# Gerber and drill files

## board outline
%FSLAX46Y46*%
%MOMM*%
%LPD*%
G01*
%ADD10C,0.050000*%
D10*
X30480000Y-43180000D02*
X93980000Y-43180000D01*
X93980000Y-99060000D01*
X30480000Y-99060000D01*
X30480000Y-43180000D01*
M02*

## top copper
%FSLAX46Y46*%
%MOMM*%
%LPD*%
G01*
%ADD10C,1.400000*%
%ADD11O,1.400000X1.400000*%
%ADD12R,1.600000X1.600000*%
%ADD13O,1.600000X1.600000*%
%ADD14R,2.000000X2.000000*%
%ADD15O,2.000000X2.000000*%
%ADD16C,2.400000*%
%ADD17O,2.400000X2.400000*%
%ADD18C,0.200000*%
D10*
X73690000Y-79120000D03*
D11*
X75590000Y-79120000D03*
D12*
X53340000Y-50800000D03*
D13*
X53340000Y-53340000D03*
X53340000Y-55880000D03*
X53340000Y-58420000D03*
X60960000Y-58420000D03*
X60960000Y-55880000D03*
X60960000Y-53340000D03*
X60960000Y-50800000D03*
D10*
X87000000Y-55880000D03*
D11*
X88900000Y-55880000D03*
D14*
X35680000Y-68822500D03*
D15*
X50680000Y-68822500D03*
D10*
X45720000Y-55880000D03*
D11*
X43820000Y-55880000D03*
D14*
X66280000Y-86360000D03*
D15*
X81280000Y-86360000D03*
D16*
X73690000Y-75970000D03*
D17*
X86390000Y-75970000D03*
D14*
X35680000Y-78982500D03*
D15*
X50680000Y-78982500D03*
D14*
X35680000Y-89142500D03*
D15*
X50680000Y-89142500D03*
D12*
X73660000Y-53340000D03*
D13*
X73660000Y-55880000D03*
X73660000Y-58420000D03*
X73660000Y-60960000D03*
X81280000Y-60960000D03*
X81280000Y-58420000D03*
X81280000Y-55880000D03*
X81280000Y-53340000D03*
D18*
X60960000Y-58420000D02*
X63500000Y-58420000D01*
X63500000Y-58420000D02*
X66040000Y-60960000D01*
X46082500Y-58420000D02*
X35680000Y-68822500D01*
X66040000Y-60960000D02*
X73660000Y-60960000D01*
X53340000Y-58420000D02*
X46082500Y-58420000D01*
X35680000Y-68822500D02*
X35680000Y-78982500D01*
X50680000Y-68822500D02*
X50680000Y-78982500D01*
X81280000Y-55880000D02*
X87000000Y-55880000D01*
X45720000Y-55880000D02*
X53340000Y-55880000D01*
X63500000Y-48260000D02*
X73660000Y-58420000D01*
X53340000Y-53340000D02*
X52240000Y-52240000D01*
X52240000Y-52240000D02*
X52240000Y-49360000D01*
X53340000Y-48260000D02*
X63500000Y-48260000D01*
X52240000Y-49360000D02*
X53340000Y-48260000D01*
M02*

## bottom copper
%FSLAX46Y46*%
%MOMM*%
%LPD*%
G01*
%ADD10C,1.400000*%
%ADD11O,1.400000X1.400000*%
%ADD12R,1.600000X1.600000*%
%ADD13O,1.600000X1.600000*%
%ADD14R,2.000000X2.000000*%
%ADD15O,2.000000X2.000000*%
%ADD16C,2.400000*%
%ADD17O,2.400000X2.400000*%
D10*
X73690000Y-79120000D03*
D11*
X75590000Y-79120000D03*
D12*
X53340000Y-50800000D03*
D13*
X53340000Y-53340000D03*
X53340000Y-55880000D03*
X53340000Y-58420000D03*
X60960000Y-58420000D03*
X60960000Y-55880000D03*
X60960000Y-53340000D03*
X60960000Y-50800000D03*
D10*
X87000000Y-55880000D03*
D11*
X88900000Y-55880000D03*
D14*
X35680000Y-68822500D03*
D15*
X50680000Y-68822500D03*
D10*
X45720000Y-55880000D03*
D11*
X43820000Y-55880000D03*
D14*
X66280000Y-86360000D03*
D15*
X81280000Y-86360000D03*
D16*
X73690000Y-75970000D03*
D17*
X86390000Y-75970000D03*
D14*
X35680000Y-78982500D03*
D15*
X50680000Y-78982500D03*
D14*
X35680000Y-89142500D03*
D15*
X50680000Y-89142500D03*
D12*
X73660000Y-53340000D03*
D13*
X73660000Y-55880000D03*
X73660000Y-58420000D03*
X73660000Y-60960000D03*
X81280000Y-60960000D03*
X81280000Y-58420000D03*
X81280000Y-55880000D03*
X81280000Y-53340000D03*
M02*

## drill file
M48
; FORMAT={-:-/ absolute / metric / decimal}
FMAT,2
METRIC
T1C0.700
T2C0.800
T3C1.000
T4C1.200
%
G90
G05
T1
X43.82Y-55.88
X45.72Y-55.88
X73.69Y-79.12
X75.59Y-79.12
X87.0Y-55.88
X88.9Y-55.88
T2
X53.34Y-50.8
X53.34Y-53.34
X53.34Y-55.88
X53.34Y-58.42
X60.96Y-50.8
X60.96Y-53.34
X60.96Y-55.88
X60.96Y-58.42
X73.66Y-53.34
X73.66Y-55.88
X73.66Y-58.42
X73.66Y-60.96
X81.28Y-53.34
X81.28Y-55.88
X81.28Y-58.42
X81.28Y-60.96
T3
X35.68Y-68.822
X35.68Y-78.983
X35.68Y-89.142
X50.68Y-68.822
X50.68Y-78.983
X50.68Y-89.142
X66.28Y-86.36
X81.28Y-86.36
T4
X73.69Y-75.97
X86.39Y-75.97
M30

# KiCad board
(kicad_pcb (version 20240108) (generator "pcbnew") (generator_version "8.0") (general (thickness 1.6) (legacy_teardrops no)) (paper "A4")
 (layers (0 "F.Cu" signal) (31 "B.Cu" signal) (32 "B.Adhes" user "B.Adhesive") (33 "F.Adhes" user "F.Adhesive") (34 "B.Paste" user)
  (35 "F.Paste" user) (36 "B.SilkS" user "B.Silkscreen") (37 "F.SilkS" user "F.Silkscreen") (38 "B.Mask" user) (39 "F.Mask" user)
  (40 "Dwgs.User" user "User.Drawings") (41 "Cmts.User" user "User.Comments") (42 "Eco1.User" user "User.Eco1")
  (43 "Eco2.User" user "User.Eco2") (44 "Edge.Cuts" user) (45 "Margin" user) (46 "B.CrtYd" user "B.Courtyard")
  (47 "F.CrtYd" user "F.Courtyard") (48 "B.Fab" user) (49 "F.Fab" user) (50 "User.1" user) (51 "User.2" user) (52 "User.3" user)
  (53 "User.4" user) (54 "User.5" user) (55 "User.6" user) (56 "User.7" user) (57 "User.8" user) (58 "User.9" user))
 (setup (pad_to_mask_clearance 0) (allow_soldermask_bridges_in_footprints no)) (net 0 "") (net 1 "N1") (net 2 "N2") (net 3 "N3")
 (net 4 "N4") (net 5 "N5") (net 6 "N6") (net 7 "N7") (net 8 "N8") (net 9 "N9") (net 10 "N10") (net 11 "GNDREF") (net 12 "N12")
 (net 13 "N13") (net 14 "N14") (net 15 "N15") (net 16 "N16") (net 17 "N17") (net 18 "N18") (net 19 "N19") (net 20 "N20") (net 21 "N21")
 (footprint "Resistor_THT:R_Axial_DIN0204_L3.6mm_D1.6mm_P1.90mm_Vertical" (layer "F.Cu") (at 73.69 79.12)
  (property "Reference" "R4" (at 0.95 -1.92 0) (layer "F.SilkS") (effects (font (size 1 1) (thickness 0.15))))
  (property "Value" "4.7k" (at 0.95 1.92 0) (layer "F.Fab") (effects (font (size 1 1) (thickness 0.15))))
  (pad "1" thru_hole circle (at 0 0) (size 1.4 1.4) (drill 0.7) (layers "*.Cu" "*.Mask") (remove_unused_layers no) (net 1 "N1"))
  (pad "2" thru_hole oval (at 1.9 0) (size 1.4 1.4) (drill 0.7) (layers "*.Cu" "*.Mask") (remove_unused_layers no) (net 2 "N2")))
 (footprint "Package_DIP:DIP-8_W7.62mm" (layer "F.Cu") (at 53.34 50.8)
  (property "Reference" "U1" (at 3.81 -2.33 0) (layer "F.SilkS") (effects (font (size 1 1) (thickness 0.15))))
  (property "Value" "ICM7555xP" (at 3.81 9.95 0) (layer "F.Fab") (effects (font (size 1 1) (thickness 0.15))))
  (pad "1" thru_hole rect (at 0 0) (size 1.6 1.6) (drill 0.8) (layers "*.Cu" "*.Mask") (remove_unused_layers no) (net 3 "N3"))
  (pad "2" thru_hole oval (at 0 2.54) (size 1.6 1.6) (drill 0.8) (layers "*.Cu" "*.Mask") (remove_unused_layers no) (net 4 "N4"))
  (pad "3" thru_hole oval (at 0 5.08) (size 1.6 1.6) (drill 0.8) (layers "*.Cu" "*.Mask") (remove_unused_layers no) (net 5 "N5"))
  (pad "4" thru_hole oval (at 0 7.62) (size 1.6 1.6) (drill 0.8) (layers "*.Cu" "*.Mask") (remove_unused_layers no) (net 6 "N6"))
  (pad "5" thru_hole oval (at 7.62 7.62) (size 1.6 1.6) (drill 0.8) (layers "*.Cu" "*.Mask") (remove_unused_layers no) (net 6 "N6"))
  (pad "6" thru_hole oval (at 7.62 5.08) (size 1.6 1.6) (drill 0.8) (layers "*.Cu" "*.Mask") (remove_unused_layers no) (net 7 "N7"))
  (pad "7" thru_hole oval (at 7.62 2.54) (size 1.6 1.6) (drill 0.8) (layers "*.Cu" "*.Mask") (remove_unused_layers no) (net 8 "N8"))
  (pad "8" thru_hole oval (at 7.62 0) (size 1.6 1.6) (drill 0.8) (layers "*.Cu" "*.Mask") (remove_unused_layers no) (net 6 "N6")))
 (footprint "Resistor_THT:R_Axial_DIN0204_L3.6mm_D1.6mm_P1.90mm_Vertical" (layer "F.Cu") (at 87 55.88)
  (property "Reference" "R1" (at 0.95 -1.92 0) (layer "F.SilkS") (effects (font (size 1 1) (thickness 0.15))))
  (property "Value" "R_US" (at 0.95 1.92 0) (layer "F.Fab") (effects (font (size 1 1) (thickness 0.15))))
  (pad "1" thru_hole circle (at 0 0) (size 1.4 1.4) (drill 0.7) (layers "*.Cu" "*.Mask") (remove_unused_layers no) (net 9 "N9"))
  (pad "2" thru_hole oval (at 1.9 0) (size 1.4 1.4) (drill 0.7) (layers "*.Cu" "*.Mask") (remove_unused_layers no) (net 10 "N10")))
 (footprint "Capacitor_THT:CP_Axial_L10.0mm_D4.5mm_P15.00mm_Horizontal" (layer "F.Cu") (at 35.68 68.8225)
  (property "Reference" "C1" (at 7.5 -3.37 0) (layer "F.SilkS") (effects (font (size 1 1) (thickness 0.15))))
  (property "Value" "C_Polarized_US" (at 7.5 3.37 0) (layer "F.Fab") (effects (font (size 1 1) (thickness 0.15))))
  (pad "1" thru_hole rect (at 0 0) (size 2 2) (drill 1) (layers "*.Cu" "*.Mask") (remove_unused_layers no) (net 6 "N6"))
  (pad "2" thru_hole oval (at 15 0) (size 2 2) (drill 1) (layers "*.Cu" "*.Mask") (remove_unused_layers no) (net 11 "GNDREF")))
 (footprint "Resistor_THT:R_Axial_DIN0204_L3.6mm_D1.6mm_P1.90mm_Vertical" (layer "F.Cu") (at 45.72 55.88 180)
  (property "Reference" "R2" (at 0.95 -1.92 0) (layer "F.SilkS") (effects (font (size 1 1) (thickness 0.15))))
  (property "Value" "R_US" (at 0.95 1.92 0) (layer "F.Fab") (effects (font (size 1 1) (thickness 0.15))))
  (pad "1" thru_hole circle (at 0 0 180) (size 1.4 1.4) (drill 0.7) (layers "*.Cu" "*.Mask") (remove_unused_layers no) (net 5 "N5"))
  (pad "2" thru_hole oval (at 1.9 0 180) (size 1.4 1.4) (drill 0.7) (layers "*.Cu" "*.Mask") (remove_unused_layers no) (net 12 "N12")))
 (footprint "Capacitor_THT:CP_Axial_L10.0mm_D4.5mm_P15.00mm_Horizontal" (layer "F.Cu") (at 66.28 86.36)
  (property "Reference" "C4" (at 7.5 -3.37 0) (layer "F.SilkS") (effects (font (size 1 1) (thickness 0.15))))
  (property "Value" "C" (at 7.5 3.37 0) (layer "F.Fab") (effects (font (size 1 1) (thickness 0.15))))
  (pad "1" thru_hole rect (at 0 0) (size 2 2) (drill 1) (layers "*.Cu" "*.Mask") (remove_unused_layers no) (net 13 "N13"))
  (pad "2" thru_hole oval (at 15 0) (size 2 2) (drill 1) (layers "*.Cu" "*.Mask") (remove_unused_layers no) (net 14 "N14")))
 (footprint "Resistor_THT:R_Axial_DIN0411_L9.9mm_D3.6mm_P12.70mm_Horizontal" (layer "F.Cu") (at 73.69 75.97)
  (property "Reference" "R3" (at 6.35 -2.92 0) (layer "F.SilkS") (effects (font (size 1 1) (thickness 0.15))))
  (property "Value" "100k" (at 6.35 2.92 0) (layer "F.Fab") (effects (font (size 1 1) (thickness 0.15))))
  (pad "1" thru_hole circle (at 0 0) (size 2.4 2.4) (drill 1.2) (layers "*.Cu" "*.Mask") (remove_unused_layers no) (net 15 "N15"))
  (pad "2" thru_hole oval (at 12.7 0) (size 2.4 2.4) (drill 1.2) (layers "*.Cu" "*.Mask") (remove_unused_layers no) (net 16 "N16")))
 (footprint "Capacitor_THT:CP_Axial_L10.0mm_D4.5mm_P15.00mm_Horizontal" (layer "F.Cu") (at 35.68 78.9825)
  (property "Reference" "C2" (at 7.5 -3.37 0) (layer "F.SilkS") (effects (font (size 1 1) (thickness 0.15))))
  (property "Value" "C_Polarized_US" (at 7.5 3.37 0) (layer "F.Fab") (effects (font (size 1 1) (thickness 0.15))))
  (pad "1" thru_hole rect (at 0 0) (size 2 2) (drill 1) (layers "*.Cu" "*.Mask") (remove_unused_layers no) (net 6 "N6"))
  (pad "2" thru_hole oval (at 15 0) (size 2 2) (drill 1) (layers "*.Cu" "*.Mask") (remove_unused_layers no) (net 11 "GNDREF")))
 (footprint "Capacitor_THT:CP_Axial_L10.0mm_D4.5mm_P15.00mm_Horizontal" (layer "F.Cu") (at 35.68 89.1425)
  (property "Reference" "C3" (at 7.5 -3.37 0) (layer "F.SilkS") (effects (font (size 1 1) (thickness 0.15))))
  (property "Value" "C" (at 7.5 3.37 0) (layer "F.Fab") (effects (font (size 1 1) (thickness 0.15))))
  (pad "1" thru_hole rect (at 0 0) (size 2 2) (drill 1) (layers "*.Cu" "*.Mask") (remove_unused_layers no) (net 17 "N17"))
  (pad "2" thru_hole oval (at 15 0) (size 2 2) (drill 1) (layers "*.Cu" "*.Mask") (remove_unused_layers no) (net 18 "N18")))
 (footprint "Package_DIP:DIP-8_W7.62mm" (layer "F.Cu") (at 73.66 53.34)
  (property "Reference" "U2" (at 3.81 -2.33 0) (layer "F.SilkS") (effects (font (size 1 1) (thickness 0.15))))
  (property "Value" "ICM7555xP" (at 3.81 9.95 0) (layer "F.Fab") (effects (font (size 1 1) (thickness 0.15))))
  (pad "1" thru_hole rect (at 0 0) (size 1.6 1.6) (drill 0.8) (layers "*.Cu" "*.Mask") (remove_unused_layers no) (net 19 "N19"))
  (pad "2" thru_hole oval (at 0 2.54) (size 1.6 1.6) (drill 0.8) (layers "*.Cu" "*.Mask") (remove_unused_layers no) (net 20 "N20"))
  (pad "3" thru_hole oval (at 0 5.08) (size 1.6 1.6) (drill 0.8) (layers "*.Cu" "*.Mask") (remove_unused_layers no) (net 4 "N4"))
  (pad "4" thru_hole oval (at 0 7.62) (size 1.6 1.6) (drill 0.8) (layers "*.Cu" "*.Mask") (remove_unused_layers no) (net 6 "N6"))
  (pad "5" thru_hole oval (at 7.62 7.62) (size 1.6 1.6) (drill 0.8) (layers "*.Cu" "*.Mask") (remove_unused_layers no) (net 6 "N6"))
  (pad "6" thru_hole oval (at 7.62 5.08) (size 1.6 1.6) (drill 0.8) (layers "*.Cu" "*.Mask") (remove_unused_layers no) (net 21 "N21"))
  (pad "7" thru_hole oval (at 7.62 2.54) (size 1.6 1.6) (drill 0.8) (layers "*.Cu" "*.Mask") (remove_unused_layers no) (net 9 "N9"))
  (pad "8" thru_hole oval (at 7.62 0) (size 1.6 1.6) (drill 0.8) (layers "*.Cu" "*.Mask") (remove_unused_layers no) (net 6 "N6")))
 (gr_rect (start 30.48 43.18) (end 93.98 99.06) (stroke (width 0.05) (type default)) (fill none) (layer "Edge.Cuts"))
 (segment (start 60.96 58.42) (end 63.5 58.42) (width 0.2) (layer "F.Cu") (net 6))
 (segment (start 63.5 58.42) (end 66.04 60.96) (width 0.2) (layer "F.Cu") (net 6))
 (segment (start 46.0825 58.42) (end 35.68 68.8225) (width 0.2) (layer "F.Cu") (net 6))
 (segment (start 66.04 60.96) (end 73.66 60.96) (width 0.2) (layer "F.Cu") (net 6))
 (segment (start 53.34 58.42) (end 46.0825 58.42) (width 0.2) (layer "F.Cu") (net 6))
 (segment (start 35.68 68.8225) (end 35.68 78.9825) (width 0.2) (layer "F.Cu") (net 6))
 (segment (start 50.68 68.8225) (end 50.68 78.9825) (width 0.2) (layer "F.Cu") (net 11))
 (segment (start 81.28 55.88) (end 87 55.88) (width 0.2) (layer "F.Cu") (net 9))
 (segment (start 45.72 55.88) (end 53.34 55.88) (width 0.2) (layer "F.Cu") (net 5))
 (segment (start 63.5 48.26) (end 73.66 58.42) (width 0.2) (layer "F.Cu") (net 4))
 (segment (start 53.34 53.34) (end 52.24 52.24) (width 0.2) (layer "F.Cu") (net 4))
 (segment (start 52.24 52.24) (end 52.24 49.36) (width 0.2) (layer "F.Cu") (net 4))
 (segment (start 53.34 48.26) (end 63.5 48.26) (width 0.2) (layer "F.Cu") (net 4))
 (segment (start 52.24 49.36) (end 53.34 48.26) (width 0.2) (layer "F.Cu") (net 4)))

